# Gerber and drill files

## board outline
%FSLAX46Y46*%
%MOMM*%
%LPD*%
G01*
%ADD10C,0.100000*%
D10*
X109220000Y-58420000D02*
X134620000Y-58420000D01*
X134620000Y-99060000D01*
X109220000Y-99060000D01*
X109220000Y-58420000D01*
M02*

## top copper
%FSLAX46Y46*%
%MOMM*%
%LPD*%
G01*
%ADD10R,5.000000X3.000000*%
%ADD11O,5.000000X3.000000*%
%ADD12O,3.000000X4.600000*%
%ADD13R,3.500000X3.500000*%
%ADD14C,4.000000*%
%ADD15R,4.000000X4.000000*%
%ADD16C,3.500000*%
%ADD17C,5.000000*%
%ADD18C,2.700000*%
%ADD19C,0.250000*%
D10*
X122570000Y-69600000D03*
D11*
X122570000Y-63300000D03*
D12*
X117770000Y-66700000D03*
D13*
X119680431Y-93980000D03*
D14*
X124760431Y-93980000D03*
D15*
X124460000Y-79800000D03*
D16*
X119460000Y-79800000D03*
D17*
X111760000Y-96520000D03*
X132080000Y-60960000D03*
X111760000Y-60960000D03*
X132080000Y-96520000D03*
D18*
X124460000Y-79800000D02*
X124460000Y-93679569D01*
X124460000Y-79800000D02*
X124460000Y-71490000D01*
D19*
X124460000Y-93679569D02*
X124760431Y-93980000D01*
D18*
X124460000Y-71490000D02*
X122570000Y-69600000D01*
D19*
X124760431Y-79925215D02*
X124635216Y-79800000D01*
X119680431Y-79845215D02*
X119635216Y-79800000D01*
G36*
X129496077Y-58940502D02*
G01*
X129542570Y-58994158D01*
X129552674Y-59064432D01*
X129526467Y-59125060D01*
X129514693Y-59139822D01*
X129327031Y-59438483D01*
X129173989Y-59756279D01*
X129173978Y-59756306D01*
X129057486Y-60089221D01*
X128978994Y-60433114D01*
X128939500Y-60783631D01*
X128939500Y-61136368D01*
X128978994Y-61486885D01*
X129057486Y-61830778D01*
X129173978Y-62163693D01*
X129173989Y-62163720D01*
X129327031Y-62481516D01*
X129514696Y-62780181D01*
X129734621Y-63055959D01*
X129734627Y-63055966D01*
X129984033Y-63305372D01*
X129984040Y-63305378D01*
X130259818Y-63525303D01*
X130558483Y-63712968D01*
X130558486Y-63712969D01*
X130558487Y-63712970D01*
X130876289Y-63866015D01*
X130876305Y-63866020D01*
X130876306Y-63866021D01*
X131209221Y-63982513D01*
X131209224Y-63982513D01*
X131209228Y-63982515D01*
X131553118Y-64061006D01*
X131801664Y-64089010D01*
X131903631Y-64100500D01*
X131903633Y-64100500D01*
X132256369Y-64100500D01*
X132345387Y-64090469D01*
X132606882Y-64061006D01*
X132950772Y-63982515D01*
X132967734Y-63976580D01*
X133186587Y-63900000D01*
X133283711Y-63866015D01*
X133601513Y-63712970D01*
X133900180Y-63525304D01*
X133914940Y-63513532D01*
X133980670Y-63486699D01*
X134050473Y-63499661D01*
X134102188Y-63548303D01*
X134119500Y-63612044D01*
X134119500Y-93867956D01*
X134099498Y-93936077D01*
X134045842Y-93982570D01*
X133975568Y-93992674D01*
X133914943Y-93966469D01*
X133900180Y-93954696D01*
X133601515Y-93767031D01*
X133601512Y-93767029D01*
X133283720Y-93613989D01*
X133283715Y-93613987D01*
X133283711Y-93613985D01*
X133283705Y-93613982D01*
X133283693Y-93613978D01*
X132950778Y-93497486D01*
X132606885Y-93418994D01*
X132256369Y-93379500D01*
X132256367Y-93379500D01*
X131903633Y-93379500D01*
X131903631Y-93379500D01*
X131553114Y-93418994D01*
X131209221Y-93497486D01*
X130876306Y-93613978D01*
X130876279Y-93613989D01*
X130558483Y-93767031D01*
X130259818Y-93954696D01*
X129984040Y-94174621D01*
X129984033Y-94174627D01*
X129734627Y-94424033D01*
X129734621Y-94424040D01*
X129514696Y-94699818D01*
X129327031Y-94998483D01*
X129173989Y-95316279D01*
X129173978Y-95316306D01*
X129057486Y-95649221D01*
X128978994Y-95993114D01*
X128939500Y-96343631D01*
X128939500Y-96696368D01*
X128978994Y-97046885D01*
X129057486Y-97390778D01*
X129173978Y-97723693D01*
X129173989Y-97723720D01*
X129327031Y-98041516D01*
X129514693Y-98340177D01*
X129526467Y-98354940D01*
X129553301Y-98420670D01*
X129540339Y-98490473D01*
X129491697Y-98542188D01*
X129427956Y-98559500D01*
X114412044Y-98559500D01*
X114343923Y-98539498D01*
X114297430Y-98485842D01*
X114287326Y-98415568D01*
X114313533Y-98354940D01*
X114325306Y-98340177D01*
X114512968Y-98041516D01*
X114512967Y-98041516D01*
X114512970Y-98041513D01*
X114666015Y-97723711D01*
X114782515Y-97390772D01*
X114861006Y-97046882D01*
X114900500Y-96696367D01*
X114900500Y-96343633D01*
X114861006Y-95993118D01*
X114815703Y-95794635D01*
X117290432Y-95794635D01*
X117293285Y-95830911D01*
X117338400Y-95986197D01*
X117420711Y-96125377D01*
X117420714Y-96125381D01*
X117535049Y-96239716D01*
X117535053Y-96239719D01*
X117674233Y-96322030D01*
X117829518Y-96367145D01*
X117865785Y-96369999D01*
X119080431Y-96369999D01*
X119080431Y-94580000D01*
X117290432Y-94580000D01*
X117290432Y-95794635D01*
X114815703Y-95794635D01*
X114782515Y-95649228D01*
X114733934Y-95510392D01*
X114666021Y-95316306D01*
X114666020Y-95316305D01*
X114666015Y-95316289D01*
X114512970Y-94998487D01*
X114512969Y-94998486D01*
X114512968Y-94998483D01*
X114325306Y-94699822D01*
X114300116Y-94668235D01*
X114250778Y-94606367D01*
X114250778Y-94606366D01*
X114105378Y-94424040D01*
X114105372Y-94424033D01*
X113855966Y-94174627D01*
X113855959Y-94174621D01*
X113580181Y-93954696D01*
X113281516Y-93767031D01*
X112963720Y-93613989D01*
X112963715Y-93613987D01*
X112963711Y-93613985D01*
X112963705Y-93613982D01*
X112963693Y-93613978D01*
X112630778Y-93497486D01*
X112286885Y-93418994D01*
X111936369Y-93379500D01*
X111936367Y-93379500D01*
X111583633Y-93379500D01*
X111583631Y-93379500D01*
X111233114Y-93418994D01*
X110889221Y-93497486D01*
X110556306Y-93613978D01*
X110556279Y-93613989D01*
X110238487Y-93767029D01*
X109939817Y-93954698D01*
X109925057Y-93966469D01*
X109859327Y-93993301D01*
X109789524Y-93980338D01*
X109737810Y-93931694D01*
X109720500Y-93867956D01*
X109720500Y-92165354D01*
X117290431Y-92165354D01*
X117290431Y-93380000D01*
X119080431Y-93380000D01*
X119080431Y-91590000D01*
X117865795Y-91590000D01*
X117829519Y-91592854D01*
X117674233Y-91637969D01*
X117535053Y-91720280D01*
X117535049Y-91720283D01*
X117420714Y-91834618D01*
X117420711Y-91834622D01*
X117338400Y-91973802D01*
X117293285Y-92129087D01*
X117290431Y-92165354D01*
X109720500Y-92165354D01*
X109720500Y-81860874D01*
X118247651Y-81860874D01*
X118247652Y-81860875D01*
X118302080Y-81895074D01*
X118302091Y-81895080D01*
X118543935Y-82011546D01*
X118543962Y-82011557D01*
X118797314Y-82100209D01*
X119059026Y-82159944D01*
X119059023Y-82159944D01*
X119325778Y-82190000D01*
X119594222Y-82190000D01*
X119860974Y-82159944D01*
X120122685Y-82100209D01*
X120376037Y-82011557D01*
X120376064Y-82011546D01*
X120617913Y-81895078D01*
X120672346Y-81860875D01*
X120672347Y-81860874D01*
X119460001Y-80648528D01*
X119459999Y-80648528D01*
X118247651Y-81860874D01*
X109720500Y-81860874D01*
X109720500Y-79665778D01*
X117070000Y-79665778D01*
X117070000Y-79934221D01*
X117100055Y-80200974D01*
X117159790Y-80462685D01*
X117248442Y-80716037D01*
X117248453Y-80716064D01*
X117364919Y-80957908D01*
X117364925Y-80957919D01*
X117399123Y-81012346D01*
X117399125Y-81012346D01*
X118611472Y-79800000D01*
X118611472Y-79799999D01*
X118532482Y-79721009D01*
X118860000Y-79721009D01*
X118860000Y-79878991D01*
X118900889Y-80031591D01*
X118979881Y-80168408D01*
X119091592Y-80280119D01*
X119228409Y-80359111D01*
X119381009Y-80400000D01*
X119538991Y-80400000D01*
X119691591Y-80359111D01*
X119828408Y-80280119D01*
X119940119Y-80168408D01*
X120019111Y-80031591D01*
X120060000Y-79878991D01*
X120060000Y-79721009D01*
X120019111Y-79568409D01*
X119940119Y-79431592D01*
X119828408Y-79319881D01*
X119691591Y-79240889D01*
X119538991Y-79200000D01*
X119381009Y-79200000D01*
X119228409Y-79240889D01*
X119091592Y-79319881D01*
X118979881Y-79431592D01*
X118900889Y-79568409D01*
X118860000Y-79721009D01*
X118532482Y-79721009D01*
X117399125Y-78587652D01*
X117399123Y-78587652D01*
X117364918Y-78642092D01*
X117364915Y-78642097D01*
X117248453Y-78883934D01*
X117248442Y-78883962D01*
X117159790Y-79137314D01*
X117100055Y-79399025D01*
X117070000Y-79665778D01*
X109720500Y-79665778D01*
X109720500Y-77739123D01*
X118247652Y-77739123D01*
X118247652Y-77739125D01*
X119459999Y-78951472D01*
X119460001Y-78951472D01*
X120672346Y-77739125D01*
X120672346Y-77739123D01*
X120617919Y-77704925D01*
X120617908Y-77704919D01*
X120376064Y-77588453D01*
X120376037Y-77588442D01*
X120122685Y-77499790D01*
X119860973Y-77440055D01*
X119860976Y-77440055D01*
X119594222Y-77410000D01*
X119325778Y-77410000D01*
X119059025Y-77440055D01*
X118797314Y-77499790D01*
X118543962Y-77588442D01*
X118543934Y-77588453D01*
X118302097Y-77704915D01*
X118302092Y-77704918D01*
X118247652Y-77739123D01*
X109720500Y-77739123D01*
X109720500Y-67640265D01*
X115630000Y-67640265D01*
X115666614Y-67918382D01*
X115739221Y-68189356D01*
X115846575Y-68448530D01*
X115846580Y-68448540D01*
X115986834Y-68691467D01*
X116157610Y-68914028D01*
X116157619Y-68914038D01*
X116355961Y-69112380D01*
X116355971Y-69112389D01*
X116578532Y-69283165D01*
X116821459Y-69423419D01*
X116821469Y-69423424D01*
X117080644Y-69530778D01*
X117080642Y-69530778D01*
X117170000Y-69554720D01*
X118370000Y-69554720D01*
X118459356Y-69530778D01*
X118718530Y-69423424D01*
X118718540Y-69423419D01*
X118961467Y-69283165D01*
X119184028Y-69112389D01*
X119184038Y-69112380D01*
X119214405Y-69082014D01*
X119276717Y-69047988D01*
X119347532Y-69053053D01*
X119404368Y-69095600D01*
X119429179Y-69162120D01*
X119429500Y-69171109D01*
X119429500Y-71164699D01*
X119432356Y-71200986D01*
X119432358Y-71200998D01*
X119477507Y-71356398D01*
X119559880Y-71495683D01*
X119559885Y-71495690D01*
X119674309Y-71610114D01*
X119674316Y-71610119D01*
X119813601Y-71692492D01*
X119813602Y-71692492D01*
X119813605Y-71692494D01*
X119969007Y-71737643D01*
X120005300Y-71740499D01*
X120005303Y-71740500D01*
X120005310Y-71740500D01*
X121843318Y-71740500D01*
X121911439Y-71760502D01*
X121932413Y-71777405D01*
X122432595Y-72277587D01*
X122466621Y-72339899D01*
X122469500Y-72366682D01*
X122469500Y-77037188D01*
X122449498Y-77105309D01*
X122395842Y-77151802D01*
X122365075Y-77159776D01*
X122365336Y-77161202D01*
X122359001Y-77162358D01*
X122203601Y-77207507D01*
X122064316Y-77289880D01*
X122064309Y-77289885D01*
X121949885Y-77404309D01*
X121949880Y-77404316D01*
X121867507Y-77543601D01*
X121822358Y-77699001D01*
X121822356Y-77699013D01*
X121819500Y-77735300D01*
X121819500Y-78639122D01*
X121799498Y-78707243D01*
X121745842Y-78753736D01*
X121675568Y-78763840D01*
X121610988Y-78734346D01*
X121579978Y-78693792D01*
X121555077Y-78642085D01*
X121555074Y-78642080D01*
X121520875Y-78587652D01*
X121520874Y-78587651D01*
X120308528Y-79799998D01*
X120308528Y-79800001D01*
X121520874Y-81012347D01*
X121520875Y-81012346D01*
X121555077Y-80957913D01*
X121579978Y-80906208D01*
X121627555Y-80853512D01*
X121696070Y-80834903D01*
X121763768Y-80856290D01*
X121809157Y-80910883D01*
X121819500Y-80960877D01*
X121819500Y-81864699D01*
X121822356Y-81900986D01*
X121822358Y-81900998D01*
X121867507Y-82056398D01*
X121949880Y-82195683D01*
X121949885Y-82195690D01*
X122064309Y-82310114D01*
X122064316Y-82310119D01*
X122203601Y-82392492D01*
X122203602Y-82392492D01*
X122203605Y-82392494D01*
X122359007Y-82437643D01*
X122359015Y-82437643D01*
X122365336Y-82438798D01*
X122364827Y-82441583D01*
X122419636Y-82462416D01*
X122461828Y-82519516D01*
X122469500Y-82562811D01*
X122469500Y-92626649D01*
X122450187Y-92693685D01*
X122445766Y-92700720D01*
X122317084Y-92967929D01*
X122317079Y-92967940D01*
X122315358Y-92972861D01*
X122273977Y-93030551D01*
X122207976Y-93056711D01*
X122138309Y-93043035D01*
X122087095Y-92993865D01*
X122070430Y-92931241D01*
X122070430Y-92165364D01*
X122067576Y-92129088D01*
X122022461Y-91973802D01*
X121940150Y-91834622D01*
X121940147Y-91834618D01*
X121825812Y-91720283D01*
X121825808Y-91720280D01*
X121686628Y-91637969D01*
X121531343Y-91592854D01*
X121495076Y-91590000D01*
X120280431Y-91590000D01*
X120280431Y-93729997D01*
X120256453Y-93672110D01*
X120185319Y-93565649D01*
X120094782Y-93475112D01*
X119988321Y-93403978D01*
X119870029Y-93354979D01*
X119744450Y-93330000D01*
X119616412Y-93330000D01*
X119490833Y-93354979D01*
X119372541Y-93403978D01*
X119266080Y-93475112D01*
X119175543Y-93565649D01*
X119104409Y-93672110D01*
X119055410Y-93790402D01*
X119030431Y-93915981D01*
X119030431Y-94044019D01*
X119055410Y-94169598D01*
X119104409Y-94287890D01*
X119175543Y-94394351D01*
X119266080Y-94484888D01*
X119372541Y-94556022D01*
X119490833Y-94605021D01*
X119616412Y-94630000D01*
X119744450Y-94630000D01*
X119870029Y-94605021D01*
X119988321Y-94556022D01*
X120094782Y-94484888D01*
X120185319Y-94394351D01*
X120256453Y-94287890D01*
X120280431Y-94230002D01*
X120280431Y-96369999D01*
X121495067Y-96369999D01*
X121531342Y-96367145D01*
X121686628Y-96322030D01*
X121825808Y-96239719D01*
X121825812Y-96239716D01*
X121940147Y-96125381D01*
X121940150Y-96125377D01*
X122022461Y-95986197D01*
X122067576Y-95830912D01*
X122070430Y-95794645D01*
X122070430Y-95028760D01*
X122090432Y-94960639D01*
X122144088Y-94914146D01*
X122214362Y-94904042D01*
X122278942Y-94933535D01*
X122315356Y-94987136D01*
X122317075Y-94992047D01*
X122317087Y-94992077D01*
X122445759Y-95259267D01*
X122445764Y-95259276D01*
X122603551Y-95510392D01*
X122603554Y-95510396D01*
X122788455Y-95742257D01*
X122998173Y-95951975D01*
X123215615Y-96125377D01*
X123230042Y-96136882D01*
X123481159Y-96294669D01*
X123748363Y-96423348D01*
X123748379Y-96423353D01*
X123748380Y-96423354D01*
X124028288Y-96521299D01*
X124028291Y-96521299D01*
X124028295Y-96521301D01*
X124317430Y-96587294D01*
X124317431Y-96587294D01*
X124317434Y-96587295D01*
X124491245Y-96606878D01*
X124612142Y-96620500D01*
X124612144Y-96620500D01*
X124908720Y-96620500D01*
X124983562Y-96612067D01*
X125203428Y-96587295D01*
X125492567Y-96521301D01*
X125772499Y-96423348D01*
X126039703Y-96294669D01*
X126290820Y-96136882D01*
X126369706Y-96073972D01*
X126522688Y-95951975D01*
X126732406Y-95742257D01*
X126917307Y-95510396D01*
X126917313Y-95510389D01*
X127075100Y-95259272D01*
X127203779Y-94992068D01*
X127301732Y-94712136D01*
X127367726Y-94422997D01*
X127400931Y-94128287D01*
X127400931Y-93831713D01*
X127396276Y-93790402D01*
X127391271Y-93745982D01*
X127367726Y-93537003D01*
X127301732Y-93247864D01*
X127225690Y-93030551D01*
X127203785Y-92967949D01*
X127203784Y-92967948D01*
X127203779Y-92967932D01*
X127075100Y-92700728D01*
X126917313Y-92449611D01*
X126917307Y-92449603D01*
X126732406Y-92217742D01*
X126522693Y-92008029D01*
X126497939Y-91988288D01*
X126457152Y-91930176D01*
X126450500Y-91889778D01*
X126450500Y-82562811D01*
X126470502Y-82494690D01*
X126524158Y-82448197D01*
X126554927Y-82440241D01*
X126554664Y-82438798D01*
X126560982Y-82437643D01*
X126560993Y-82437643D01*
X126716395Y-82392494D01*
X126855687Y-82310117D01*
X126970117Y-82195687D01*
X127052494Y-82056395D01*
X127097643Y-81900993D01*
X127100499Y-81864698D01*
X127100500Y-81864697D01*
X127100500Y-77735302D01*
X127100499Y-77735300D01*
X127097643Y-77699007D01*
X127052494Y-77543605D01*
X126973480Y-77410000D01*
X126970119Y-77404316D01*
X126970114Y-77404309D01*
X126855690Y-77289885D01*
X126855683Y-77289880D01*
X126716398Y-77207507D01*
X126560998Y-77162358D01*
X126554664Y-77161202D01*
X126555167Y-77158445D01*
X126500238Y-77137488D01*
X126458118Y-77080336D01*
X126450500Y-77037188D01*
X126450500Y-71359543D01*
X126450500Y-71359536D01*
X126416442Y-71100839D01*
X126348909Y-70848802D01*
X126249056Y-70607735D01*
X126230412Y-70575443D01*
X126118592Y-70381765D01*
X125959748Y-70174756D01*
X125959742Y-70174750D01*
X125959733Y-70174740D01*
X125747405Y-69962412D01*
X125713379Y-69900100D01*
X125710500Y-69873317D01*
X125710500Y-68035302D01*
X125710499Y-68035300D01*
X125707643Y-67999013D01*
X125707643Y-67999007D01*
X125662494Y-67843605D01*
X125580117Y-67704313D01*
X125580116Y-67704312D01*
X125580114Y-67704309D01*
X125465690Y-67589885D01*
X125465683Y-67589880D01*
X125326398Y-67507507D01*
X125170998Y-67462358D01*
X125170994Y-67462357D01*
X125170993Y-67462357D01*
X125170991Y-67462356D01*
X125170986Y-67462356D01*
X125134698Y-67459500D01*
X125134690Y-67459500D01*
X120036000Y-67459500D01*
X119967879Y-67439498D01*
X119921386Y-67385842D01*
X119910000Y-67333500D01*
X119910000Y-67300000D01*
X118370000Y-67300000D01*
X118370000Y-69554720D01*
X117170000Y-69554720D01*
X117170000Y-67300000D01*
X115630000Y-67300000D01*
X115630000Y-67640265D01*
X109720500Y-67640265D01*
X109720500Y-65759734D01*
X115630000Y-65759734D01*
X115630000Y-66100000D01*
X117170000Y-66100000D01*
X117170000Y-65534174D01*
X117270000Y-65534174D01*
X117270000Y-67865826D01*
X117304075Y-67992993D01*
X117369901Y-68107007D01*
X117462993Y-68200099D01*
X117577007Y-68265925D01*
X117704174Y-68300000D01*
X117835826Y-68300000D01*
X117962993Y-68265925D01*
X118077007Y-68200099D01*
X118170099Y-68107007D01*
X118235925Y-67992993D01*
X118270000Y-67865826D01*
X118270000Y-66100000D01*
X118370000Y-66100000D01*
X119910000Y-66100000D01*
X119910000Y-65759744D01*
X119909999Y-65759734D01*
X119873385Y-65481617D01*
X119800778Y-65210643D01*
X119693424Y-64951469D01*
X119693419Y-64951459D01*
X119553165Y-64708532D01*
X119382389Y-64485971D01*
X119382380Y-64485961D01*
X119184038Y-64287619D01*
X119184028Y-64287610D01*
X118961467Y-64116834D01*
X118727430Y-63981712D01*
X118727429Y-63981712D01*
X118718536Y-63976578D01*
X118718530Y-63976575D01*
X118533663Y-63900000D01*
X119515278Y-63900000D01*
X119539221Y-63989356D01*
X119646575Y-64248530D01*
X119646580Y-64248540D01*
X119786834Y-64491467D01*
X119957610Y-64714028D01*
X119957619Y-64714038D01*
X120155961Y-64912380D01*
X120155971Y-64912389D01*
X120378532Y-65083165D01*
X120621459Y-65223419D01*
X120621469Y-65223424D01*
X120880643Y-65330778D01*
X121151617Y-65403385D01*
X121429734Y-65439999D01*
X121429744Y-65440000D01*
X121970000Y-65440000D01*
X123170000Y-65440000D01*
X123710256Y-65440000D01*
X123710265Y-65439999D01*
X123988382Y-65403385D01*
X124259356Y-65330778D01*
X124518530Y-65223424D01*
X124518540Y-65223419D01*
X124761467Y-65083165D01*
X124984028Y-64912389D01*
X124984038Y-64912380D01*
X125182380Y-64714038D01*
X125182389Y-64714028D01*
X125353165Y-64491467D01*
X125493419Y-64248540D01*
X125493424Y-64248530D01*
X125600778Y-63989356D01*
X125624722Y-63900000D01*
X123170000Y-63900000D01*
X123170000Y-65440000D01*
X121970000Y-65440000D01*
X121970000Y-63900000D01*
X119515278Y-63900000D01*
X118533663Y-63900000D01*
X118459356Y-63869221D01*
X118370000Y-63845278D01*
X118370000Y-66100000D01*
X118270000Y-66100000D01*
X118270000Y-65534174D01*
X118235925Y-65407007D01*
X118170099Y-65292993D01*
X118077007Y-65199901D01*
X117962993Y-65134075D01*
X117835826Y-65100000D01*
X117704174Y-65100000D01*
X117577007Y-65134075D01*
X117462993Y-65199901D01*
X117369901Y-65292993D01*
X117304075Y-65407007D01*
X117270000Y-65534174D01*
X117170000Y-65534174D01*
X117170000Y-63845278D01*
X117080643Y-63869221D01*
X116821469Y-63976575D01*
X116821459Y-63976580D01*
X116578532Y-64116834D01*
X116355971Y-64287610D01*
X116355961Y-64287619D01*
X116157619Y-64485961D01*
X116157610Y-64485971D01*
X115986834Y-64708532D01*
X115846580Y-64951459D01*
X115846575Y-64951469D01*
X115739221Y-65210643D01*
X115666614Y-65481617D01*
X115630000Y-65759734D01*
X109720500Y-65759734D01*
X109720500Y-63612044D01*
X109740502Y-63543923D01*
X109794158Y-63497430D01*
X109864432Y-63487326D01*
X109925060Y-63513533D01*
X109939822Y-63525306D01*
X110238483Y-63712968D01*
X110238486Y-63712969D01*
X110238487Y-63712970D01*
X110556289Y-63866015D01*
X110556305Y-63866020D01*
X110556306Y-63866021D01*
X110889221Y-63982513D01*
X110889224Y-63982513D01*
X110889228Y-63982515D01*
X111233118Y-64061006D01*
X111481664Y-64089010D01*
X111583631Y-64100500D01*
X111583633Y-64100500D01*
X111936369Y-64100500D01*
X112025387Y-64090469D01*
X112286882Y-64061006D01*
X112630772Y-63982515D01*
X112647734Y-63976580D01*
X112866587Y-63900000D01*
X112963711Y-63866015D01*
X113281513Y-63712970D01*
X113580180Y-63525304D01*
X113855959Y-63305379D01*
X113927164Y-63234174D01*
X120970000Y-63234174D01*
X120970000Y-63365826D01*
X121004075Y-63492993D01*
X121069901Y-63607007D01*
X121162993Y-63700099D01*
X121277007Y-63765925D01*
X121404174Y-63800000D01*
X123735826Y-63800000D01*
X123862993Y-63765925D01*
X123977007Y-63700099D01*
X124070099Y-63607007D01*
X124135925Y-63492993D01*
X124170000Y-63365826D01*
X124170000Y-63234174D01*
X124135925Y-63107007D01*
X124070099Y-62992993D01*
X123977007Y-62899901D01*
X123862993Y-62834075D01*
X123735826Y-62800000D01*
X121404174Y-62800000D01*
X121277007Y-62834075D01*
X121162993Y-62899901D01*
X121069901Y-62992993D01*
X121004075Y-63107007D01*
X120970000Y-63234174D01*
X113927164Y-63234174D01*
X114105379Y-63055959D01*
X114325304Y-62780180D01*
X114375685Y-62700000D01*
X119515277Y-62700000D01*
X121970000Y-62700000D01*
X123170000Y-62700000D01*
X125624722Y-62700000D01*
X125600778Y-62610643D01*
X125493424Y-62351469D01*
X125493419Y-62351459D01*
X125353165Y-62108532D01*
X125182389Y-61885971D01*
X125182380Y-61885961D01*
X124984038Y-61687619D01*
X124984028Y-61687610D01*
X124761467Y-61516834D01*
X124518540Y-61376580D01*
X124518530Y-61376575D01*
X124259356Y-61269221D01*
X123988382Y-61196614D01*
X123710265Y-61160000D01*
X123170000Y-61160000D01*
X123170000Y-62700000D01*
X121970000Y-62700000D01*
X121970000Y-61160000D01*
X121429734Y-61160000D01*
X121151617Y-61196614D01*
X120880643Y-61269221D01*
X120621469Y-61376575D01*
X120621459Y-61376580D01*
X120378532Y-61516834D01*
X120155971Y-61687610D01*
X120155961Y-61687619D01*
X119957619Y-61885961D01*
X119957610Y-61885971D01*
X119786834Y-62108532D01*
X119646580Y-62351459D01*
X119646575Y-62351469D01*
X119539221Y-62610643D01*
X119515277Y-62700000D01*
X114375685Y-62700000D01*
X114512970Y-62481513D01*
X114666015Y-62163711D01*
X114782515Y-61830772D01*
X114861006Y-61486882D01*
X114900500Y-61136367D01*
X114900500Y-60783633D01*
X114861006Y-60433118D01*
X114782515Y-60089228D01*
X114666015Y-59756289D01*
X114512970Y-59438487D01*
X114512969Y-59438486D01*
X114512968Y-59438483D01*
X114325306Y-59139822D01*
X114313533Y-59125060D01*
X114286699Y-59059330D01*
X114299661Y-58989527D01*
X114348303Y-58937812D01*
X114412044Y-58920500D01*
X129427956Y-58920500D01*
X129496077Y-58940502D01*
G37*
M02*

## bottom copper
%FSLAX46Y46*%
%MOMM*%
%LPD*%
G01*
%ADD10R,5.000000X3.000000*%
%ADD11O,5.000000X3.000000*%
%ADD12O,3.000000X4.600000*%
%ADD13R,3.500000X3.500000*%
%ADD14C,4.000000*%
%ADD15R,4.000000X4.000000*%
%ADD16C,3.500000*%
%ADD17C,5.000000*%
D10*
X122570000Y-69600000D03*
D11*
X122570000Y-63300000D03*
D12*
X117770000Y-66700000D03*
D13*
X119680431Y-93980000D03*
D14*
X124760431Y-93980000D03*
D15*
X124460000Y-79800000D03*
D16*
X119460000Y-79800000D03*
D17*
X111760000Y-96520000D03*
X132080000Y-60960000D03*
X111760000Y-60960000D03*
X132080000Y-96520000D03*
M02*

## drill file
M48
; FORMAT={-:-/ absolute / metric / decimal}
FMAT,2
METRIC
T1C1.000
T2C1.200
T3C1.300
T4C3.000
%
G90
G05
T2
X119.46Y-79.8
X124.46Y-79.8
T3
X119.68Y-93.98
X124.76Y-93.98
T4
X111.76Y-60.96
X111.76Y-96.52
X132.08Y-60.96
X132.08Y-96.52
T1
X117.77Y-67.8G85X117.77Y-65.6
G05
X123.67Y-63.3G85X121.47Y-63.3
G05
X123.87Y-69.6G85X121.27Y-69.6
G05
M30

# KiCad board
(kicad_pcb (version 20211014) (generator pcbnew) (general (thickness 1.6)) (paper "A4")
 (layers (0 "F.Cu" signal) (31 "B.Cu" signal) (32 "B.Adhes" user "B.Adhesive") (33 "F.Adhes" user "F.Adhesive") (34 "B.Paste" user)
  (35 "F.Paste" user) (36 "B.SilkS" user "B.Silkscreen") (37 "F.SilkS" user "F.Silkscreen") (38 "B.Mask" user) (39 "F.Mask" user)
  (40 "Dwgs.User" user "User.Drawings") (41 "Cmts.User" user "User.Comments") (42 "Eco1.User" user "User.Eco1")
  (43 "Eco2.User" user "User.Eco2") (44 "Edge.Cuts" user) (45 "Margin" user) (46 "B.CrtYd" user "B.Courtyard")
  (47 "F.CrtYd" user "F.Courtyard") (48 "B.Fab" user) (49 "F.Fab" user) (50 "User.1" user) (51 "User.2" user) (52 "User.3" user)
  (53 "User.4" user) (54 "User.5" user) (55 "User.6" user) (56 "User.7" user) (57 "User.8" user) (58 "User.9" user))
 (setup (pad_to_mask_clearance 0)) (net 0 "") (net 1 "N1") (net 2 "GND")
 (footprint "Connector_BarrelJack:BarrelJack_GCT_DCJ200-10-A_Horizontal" (layer "F.Cu") (at 122.57 69.6 180)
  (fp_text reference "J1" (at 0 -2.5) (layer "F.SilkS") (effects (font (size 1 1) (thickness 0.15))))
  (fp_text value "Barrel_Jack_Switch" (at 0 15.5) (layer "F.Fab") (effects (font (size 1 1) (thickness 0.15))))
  (pad "1" thru_hole rect (at 0 0 180) (size 5 3) (drill oval 3.6 1) (layers *.Cu *.Mask) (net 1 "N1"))
  (pad "2" thru_hole oval (at 0 6.3 180) (size 5 3) (drill oval 3.2 1) (layers *.Cu *.Mask) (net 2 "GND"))
  (pad "3" thru_hole oval (at 4.8 2.9 180) (size 3 4.6) (drill oval 1 3.2) (layers *.Cu *.Mask) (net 2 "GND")))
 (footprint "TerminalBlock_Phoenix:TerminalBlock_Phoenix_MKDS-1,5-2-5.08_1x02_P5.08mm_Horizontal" (layer "F.Cu") (at 119.680431 93.98)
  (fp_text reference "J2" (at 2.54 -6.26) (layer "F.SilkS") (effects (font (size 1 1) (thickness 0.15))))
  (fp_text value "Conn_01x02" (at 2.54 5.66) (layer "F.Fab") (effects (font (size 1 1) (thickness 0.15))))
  (pad "1" thru_hole rect (at 0 0) (size 3.5 3.5) (drill 1.3) (layers *.Cu *.Mask) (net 2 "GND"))
  (pad "2" thru_hole circle (at 5.08 0) (size 4 4) (drill 1.3) (layers *.Cu *.Mask) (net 1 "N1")))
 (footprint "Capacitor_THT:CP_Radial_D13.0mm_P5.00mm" (layer "F.Cu") (at 124.46 79.8 180)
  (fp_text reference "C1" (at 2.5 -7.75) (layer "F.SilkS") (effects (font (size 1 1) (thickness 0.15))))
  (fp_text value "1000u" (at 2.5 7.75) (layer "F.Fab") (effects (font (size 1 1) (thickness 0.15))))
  (pad "1" thru_hole rect (at 0 0 180) (size 4 4) (drill 1.2) (layers *.Cu *.Mask) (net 1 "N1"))
  (pad "2" thru_hole circle (at 5 0 180) (size 3.5 3.5) (drill 1.2) (layers *.Cu *.Mask) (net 2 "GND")))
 (gr_rect (start 109.22 58.42) (end 134.62 99.06) (layer "Edge.Cuts") (width 0.1) (fill none))
 (via (at 111.76 96.52) (size 5) (drill 3) (layers "F.Cu" "B.Cu") (free) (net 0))
 (via (at 132.08 60.96) (size 5) (drill 3) (layers "F.Cu" "B.Cu") (free) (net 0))
 (via (at 111.76 60.96) (size 5) (drill 3) (layers "F.Cu" "B.Cu") (free) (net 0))
 (via (at 132.08 96.52) (size 5) (drill 3) (layers "F.Cu" "B.Cu") (free) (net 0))
 (segment (start 124.46 79.8) (end 124.46 93.679569) (width 2.7) (layer "F.Cu") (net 1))
 (segment (start 124.46 79.8) (end 124.46 71.49) (width 2.7) (layer "F.Cu") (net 1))
 (segment (start 124.46 93.679569) (end 124.760431 93.98) (width 0.25) (layer "F.Cu") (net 1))
 (segment (start 124.46 71.49) (end 122.57 69.6) (width 2.7) (layer "F.Cu") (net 1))
 (segment (start 124.760431 79.925215) (end 124.635216 79.8) (width 0.25) (layer "F.Cu") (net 1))
 (segment (start 119.680431 79.845215) (end 119.635216 79.8) (width 0.25) (layer "F.Cu") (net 2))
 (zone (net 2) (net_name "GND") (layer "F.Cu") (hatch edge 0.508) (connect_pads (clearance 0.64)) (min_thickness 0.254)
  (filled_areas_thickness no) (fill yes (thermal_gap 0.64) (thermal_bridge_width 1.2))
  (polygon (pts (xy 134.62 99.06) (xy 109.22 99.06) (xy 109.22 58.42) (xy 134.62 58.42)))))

